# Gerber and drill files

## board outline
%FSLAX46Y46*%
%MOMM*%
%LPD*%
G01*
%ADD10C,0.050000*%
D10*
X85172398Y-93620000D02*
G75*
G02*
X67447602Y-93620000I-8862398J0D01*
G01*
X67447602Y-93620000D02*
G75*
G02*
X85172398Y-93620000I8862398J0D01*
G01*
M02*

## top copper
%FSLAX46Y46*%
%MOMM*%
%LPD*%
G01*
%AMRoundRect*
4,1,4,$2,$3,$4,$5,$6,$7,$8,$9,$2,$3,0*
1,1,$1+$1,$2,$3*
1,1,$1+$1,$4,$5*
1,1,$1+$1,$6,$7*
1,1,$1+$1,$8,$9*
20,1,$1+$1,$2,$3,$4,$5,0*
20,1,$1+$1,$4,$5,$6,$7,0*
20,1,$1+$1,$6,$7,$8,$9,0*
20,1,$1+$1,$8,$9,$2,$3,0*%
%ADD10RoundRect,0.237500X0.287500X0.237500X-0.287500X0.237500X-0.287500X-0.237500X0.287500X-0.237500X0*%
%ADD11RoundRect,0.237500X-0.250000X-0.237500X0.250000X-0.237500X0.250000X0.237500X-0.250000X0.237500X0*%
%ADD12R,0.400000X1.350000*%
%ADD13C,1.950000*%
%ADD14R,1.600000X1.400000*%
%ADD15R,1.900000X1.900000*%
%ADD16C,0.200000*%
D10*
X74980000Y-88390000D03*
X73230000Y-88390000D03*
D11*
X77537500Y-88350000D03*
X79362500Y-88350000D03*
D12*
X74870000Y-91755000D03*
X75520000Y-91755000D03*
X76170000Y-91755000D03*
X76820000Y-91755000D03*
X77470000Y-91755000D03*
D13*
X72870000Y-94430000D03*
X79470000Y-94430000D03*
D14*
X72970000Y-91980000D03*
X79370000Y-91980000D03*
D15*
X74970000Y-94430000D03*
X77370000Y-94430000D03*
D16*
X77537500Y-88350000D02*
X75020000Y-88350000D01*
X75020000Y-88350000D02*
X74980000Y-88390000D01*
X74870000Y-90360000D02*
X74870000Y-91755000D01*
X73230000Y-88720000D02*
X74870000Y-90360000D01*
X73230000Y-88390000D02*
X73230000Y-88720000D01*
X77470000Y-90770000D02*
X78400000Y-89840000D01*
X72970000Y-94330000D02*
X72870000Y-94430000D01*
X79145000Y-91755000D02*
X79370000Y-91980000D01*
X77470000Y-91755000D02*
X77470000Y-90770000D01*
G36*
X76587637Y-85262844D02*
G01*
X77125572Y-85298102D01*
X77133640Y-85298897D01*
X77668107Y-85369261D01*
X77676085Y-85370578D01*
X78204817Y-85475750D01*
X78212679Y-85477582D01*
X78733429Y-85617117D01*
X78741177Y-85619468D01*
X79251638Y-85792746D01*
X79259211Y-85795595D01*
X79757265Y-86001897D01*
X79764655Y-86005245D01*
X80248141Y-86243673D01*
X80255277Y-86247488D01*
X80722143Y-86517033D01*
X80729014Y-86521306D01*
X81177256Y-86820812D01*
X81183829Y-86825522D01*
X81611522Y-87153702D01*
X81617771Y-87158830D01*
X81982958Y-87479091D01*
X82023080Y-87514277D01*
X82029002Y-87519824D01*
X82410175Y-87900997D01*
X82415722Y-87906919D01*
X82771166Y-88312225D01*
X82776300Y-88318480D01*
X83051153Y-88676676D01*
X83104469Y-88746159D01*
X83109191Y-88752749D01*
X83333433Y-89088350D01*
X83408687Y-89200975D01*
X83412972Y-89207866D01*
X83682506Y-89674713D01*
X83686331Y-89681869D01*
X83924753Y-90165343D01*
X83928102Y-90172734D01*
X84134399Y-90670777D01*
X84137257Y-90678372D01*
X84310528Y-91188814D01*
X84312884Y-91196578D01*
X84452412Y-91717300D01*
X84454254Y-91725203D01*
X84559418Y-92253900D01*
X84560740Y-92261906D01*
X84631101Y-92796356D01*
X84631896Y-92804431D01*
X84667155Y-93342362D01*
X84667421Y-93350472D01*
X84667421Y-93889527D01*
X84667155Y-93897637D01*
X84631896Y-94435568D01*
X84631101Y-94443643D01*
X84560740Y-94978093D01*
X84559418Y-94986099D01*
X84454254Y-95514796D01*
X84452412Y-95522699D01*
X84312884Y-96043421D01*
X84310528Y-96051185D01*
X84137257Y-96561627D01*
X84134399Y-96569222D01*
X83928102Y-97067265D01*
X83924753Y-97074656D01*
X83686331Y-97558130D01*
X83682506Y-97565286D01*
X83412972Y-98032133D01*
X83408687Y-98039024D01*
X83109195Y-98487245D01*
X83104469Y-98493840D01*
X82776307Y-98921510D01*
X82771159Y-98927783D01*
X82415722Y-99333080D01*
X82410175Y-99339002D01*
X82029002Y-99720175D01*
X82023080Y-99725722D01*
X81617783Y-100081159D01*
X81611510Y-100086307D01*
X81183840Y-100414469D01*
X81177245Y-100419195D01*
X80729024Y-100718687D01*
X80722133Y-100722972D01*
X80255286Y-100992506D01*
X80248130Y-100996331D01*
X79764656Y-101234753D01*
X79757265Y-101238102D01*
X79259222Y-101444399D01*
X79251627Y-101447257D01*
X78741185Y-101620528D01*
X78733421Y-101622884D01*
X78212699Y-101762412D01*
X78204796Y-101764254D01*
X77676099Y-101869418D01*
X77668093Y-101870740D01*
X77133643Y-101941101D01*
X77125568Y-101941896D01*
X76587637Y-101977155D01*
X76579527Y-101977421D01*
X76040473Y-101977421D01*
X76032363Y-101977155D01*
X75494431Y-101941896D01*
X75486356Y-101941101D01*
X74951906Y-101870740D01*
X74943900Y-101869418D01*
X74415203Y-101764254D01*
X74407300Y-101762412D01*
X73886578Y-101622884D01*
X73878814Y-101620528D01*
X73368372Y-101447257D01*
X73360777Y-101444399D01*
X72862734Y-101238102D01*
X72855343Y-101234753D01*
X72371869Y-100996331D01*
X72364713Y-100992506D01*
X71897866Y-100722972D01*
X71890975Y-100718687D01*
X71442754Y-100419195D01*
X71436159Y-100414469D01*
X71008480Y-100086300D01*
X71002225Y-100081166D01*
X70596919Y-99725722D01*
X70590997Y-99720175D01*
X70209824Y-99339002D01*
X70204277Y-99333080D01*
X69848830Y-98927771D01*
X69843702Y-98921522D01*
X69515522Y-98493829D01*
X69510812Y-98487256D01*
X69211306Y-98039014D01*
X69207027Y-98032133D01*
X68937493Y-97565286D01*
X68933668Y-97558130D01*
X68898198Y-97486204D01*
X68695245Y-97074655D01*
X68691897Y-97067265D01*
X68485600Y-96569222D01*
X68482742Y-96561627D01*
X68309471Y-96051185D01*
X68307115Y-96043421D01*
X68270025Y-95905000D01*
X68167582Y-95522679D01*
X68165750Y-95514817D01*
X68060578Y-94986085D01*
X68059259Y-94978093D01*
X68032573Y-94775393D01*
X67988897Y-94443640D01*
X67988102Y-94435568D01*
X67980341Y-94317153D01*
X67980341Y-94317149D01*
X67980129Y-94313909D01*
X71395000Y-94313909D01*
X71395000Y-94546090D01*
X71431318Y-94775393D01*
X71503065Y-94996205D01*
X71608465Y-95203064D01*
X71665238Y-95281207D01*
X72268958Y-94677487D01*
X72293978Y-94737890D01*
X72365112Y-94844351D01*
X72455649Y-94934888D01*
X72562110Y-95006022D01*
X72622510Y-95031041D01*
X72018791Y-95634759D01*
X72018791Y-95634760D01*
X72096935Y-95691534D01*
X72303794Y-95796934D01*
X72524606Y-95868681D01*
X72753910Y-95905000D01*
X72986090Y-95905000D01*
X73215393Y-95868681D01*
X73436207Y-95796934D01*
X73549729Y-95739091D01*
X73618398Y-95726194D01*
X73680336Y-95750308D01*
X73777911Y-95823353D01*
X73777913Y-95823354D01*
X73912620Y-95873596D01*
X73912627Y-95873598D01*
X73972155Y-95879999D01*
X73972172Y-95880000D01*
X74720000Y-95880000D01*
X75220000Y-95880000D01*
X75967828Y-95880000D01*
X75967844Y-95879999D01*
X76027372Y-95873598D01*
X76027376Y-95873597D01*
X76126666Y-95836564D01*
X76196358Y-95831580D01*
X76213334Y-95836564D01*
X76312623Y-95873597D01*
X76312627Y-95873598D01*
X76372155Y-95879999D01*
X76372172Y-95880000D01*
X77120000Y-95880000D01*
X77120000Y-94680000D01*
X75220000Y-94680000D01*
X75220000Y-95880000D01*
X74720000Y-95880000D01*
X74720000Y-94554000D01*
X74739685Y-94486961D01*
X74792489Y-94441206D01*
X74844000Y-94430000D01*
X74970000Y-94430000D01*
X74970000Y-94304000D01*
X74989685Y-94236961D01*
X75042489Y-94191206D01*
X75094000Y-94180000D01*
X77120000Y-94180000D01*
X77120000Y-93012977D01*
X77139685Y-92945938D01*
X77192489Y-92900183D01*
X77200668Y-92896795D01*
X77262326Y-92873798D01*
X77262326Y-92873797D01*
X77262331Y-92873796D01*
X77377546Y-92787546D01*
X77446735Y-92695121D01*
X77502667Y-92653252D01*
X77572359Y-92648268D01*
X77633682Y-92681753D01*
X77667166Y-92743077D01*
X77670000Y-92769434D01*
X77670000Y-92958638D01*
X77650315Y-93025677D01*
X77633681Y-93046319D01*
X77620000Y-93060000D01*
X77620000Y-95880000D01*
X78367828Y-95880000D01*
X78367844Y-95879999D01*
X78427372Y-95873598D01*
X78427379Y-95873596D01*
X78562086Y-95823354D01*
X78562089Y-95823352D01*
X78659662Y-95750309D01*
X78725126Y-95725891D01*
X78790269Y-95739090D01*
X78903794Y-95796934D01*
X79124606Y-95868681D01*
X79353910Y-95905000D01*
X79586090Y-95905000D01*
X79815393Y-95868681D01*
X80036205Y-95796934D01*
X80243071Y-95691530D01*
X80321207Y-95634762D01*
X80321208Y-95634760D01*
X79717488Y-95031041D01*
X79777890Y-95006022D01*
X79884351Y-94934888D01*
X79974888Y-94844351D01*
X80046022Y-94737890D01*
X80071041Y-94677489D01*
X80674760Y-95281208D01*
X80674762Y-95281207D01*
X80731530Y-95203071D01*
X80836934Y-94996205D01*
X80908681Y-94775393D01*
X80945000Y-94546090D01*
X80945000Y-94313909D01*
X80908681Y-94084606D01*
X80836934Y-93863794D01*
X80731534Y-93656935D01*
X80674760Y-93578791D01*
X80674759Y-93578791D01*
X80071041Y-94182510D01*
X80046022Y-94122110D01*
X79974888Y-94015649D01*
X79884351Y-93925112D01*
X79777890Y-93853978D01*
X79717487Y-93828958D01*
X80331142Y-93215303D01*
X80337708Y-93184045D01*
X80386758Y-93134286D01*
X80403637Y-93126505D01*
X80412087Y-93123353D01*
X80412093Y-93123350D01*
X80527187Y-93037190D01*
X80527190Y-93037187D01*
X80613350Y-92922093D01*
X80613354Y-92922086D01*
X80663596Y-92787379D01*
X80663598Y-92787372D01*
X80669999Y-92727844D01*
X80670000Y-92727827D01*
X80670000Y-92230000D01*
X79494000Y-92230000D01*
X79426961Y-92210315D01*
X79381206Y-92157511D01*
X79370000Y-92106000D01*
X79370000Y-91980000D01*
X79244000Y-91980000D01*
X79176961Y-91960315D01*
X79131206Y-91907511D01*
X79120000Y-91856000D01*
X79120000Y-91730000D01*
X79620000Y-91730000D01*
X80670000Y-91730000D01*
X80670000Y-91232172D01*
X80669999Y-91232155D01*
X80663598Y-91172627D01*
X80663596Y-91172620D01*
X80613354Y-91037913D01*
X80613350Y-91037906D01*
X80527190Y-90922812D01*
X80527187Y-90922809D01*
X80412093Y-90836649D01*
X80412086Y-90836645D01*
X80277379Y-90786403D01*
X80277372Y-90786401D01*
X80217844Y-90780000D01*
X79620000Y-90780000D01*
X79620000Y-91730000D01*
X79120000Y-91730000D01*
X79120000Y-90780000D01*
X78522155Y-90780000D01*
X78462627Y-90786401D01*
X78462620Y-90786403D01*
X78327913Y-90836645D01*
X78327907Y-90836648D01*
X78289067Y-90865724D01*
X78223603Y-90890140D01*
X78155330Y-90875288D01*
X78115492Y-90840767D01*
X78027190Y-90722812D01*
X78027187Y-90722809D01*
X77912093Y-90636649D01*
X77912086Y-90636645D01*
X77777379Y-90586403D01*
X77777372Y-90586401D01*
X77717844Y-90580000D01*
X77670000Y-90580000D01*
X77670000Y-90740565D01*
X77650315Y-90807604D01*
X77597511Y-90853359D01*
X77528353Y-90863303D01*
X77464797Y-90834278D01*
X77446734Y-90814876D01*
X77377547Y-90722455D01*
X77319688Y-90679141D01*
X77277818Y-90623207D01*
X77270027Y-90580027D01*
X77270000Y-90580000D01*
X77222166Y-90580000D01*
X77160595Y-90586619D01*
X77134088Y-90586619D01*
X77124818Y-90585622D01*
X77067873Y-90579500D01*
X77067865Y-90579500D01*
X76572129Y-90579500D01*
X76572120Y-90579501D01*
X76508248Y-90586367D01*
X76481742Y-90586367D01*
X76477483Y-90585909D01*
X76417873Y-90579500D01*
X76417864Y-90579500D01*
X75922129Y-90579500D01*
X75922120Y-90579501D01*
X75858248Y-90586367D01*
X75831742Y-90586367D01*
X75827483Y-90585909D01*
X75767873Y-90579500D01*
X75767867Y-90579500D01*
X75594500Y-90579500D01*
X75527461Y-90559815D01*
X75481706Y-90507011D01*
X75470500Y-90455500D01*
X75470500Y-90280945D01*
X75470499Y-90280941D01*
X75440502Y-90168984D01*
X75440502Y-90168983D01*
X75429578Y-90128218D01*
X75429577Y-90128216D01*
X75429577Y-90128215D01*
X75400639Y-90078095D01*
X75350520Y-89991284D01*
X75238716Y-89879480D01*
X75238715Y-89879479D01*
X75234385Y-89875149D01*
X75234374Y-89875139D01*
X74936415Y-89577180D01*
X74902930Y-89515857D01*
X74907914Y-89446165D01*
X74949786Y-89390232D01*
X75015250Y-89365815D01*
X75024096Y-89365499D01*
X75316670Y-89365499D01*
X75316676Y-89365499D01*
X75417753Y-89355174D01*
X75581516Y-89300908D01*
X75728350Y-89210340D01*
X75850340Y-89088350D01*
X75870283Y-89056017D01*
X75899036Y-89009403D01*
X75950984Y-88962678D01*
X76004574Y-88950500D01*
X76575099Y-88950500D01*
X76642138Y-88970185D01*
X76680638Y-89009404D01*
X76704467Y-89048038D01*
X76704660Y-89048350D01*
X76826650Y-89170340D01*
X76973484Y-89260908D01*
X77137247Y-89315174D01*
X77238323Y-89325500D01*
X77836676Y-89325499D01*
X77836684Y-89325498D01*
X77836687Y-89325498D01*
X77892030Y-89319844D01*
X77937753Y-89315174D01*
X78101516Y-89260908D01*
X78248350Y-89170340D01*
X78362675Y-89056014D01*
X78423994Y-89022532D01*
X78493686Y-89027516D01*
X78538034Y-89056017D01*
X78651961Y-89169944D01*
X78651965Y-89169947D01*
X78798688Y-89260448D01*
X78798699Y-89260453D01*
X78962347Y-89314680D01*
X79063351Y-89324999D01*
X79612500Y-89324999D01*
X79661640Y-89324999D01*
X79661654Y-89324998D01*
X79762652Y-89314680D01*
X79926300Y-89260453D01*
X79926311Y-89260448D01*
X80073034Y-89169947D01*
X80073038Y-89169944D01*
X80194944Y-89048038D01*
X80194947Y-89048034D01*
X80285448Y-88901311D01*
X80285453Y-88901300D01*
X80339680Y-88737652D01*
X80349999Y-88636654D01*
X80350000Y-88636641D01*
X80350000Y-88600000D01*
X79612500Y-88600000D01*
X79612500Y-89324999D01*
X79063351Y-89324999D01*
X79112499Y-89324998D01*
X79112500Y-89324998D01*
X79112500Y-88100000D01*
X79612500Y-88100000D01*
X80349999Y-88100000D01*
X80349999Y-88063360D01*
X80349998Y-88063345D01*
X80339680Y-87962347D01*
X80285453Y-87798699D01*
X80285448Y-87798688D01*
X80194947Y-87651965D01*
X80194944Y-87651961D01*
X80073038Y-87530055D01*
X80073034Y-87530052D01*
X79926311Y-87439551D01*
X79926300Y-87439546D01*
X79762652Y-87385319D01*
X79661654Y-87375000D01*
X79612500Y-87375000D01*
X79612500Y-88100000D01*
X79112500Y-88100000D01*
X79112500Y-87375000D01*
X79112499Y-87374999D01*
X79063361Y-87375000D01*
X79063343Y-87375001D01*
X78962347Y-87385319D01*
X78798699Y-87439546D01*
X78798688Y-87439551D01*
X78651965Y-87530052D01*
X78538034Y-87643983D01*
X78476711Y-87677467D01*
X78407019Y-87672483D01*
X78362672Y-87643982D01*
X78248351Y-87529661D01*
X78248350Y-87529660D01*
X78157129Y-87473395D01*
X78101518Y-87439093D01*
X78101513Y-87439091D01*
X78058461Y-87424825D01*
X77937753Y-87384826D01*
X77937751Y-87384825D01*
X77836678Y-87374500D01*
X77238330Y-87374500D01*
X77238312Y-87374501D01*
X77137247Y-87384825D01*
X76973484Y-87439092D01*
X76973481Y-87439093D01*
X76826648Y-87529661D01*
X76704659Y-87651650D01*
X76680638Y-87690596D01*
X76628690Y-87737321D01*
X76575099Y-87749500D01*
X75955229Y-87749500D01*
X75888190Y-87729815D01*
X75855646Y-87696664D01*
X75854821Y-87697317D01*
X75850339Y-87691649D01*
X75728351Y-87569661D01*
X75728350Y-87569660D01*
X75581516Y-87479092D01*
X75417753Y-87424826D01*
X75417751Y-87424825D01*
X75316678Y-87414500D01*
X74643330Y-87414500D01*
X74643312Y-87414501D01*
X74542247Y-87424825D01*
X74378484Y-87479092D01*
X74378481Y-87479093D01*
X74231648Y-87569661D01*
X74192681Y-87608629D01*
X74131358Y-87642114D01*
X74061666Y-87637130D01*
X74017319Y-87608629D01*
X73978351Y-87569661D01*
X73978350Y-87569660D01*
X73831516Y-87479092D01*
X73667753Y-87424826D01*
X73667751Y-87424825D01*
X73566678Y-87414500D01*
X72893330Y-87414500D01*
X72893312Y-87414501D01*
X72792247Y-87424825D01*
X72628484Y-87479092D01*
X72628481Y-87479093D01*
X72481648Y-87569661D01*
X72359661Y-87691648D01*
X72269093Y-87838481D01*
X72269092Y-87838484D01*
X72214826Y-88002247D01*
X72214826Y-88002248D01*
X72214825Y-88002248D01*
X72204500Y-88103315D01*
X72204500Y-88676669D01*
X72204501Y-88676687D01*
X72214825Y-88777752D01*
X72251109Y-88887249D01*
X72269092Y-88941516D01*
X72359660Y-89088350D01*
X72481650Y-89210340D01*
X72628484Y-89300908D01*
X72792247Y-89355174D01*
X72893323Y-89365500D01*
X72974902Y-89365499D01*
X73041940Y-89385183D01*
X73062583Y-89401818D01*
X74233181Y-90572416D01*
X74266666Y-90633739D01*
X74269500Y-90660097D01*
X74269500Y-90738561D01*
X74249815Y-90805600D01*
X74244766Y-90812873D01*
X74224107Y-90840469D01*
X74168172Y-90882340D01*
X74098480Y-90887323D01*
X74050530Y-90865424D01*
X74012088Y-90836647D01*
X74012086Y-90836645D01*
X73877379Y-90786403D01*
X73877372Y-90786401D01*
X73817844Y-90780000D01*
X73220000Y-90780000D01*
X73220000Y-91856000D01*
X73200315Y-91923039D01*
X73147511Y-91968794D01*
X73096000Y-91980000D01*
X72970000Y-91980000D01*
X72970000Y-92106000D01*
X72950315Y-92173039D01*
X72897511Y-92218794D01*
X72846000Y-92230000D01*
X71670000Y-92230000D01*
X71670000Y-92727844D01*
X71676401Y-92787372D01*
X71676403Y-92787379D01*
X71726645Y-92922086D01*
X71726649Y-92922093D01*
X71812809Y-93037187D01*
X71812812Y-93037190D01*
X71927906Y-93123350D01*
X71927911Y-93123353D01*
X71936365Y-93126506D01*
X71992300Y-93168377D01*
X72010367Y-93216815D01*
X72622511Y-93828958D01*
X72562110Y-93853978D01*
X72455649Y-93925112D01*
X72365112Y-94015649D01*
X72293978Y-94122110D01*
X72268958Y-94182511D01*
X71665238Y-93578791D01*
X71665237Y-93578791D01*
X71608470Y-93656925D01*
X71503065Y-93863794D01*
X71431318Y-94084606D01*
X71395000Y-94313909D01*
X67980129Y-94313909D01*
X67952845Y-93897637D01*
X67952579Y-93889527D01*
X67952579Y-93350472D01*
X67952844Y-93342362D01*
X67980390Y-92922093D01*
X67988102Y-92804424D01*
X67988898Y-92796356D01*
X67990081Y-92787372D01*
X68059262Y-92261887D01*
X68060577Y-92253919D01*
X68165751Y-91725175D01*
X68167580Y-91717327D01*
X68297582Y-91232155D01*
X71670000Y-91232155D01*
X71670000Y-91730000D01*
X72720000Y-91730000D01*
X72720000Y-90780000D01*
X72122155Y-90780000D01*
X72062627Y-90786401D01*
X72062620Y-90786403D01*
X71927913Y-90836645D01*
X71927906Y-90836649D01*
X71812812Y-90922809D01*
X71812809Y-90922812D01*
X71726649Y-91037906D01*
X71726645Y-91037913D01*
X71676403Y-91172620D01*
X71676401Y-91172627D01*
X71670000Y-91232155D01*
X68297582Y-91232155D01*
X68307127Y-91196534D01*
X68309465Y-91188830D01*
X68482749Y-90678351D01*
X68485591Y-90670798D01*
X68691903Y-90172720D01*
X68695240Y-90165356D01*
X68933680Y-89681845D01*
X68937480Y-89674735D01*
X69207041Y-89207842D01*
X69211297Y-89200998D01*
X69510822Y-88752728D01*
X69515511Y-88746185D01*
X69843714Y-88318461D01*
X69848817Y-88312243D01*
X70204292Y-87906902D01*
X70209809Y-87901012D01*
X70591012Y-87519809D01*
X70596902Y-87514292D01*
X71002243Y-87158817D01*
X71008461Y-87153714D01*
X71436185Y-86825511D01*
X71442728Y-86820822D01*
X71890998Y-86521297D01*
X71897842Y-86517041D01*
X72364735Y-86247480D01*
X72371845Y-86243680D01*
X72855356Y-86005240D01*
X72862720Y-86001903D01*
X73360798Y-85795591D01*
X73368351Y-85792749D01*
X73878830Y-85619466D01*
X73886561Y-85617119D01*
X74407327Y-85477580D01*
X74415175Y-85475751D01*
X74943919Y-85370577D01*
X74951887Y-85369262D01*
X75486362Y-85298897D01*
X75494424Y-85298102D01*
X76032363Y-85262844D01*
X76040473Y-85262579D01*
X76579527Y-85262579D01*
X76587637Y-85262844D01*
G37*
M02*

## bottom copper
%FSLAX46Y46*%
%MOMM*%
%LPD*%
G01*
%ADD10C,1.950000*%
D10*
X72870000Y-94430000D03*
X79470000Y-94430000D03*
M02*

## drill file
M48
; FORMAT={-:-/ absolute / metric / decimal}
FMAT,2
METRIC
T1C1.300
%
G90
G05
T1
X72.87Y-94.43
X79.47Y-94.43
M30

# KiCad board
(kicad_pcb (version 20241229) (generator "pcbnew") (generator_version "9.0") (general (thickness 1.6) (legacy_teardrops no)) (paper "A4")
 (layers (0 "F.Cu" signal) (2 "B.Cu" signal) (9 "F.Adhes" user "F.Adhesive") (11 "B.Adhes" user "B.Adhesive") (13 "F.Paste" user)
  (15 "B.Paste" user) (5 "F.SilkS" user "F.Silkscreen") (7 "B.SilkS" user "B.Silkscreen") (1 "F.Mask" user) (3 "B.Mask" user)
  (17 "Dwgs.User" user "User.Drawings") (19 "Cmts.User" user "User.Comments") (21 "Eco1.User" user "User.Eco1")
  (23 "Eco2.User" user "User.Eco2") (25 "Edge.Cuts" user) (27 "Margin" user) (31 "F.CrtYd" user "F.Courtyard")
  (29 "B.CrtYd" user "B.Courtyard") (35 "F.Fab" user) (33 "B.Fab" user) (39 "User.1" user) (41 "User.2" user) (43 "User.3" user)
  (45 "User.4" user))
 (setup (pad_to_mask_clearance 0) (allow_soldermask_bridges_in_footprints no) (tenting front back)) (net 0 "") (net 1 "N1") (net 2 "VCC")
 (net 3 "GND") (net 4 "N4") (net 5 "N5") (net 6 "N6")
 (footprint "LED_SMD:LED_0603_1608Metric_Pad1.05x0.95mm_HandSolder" (layer "F.Cu") (at 74.105 88.39 180)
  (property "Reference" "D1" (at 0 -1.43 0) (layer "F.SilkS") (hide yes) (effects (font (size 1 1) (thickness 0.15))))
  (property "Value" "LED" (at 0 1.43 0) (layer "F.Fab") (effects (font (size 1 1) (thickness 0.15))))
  (pad "1" smd roundrect (at -0.875 0 180) (size 1.05 0.95) (layers "F.Cu" "F.Mask" "F.Paste") (roundrect_rratio 0.25) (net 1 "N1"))
  (pad "2" smd roundrect (at 0.875 0 180) (size 1.05 0.95) (layers "F.Cu" "F.Mask" "F.Paste") (roundrect_rratio 0.25) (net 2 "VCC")))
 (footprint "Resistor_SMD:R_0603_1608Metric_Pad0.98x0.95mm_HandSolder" (layer "F.Cu") (at 78.45 88.35)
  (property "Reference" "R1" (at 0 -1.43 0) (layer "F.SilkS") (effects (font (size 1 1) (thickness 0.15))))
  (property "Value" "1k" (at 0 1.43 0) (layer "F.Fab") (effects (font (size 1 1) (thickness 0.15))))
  (pad "1" smd roundrect (at -0.9125 0) (size 0.975 0.95) (layers "F.Cu" "F.Mask" "F.Paste") (roundrect_rratio 0.25) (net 1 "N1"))
  (pad "2" smd roundrect (at 0.9125 0) (size 0.975 0.95) (layers "F.Cu" "F.Mask" "F.Paste") (roundrect_rratio 0.25) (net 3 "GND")))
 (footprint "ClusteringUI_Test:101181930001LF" (layer "F.Cu") (at 76.17 94.135)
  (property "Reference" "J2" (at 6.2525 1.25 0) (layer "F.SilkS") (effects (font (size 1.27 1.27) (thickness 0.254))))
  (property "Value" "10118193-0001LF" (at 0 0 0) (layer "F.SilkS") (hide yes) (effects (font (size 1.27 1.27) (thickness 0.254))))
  (pad "1" smd rect (at -1.3 -2.38) (size 0.4 1.35) (layers "F.Cu" "F.Mask" "F.Paste") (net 2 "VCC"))
  (pad "2" smd rect (at -0.65 -2.38) (size 0.4 1.35) (layers "F.Cu" "F.Mask" "F.Paste") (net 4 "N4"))
  (pad "3" smd rect (at 0 -2.38) (size 0.4 1.35) (layers "F.Cu" "F.Mask" "F.Paste") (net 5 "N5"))
  (pad "4" smd rect (at 0.65 -2.38) (size 0.4 1.35) (layers "F.Cu" "F.Mask" "F.Paste") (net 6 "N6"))
  (pad "5" smd rect (at 1.3 -2.38) (size 0.4 1.35) (layers "F.Cu" "F.Mask" "F.Paste") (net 3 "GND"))
  (pad "MH1" thru_hole circle (at -3.3 0.295) (size 1.95 1.95) (drill 1.3) (layers "*.Cu" "*.Mask") (remove_unused_layers no) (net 3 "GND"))
  (pad "MH2" thru_hole circle (at 3.3 0.295) (size 1.95 1.95) (drill 1.3) (layers "*.Cu" "*.Mask") (remove_unused_layers no) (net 3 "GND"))
  (pad "MP1" smd rect (at -3.2 -2.155 90) (size 1.4 1.6) (layers "F.Cu" "F.Mask" "F.Paste") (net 3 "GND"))
  (pad "MP2" smd rect (at 3.2 -2.155 90) (size 1.4 1.6) (layers "F.Cu" "F.Mask" "F.Paste") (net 3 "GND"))
  (pad "MP3" smd rect (at -1.2 0.295) (size 1.9 1.9) (layers "F.Cu" "F.Mask" "F.Paste") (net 3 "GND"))
  (pad "MP4" smd rect (at 1.2 0.295) (size 1.9 1.9) (layers "F.Cu" "F.Mask" "F.Paste") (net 3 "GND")))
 (gr_circle (center 76.31 93.62) (end 83.45 98.87) (stroke (width 0.05) (type default)) (fill no) (layer "Edge.Cuts"))
 (segment (start 77.5375 88.35) (end 75.02 88.35) (width 0.2) (layer "F.Cu") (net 1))
 (segment (start 75.02 88.35) (end 74.98 88.39) (width 0.2) (layer "F.Cu") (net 1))
 (segment (start 74.87 90.36) (end 74.87 91.755) (width 0.2) (layer "F.Cu") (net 2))
 (segment (start 73.23 88.72) (end 74.87 90.36) (width 0.2) (layer "F.Cu") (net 2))
 (segment (start 73.23 88.39) (end 73.23 88.72) (width 0.2) (layer "F.Cu") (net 2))
 (segment (start 77.47 90.77) (end 78.4 89.84) (width 0.2) (layer "F.Cu") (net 3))
 (segment (start 72.97 94.33) (end 72.87 94.43) (width 0.2) (layer "F.Cu") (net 3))
 (segment (start 79.145 91.755) (end 79.37 91.98) (width 0.2) (layer "F.Cu") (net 3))
 (segment (start 77.47 91.755) (end 77.47 90.77) (width 0.2) (layer "F.Cu") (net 3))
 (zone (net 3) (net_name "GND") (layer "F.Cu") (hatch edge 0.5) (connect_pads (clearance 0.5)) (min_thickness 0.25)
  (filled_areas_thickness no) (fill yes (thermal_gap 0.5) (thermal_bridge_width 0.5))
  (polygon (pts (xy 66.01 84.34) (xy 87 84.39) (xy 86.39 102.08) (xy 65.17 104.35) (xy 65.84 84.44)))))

